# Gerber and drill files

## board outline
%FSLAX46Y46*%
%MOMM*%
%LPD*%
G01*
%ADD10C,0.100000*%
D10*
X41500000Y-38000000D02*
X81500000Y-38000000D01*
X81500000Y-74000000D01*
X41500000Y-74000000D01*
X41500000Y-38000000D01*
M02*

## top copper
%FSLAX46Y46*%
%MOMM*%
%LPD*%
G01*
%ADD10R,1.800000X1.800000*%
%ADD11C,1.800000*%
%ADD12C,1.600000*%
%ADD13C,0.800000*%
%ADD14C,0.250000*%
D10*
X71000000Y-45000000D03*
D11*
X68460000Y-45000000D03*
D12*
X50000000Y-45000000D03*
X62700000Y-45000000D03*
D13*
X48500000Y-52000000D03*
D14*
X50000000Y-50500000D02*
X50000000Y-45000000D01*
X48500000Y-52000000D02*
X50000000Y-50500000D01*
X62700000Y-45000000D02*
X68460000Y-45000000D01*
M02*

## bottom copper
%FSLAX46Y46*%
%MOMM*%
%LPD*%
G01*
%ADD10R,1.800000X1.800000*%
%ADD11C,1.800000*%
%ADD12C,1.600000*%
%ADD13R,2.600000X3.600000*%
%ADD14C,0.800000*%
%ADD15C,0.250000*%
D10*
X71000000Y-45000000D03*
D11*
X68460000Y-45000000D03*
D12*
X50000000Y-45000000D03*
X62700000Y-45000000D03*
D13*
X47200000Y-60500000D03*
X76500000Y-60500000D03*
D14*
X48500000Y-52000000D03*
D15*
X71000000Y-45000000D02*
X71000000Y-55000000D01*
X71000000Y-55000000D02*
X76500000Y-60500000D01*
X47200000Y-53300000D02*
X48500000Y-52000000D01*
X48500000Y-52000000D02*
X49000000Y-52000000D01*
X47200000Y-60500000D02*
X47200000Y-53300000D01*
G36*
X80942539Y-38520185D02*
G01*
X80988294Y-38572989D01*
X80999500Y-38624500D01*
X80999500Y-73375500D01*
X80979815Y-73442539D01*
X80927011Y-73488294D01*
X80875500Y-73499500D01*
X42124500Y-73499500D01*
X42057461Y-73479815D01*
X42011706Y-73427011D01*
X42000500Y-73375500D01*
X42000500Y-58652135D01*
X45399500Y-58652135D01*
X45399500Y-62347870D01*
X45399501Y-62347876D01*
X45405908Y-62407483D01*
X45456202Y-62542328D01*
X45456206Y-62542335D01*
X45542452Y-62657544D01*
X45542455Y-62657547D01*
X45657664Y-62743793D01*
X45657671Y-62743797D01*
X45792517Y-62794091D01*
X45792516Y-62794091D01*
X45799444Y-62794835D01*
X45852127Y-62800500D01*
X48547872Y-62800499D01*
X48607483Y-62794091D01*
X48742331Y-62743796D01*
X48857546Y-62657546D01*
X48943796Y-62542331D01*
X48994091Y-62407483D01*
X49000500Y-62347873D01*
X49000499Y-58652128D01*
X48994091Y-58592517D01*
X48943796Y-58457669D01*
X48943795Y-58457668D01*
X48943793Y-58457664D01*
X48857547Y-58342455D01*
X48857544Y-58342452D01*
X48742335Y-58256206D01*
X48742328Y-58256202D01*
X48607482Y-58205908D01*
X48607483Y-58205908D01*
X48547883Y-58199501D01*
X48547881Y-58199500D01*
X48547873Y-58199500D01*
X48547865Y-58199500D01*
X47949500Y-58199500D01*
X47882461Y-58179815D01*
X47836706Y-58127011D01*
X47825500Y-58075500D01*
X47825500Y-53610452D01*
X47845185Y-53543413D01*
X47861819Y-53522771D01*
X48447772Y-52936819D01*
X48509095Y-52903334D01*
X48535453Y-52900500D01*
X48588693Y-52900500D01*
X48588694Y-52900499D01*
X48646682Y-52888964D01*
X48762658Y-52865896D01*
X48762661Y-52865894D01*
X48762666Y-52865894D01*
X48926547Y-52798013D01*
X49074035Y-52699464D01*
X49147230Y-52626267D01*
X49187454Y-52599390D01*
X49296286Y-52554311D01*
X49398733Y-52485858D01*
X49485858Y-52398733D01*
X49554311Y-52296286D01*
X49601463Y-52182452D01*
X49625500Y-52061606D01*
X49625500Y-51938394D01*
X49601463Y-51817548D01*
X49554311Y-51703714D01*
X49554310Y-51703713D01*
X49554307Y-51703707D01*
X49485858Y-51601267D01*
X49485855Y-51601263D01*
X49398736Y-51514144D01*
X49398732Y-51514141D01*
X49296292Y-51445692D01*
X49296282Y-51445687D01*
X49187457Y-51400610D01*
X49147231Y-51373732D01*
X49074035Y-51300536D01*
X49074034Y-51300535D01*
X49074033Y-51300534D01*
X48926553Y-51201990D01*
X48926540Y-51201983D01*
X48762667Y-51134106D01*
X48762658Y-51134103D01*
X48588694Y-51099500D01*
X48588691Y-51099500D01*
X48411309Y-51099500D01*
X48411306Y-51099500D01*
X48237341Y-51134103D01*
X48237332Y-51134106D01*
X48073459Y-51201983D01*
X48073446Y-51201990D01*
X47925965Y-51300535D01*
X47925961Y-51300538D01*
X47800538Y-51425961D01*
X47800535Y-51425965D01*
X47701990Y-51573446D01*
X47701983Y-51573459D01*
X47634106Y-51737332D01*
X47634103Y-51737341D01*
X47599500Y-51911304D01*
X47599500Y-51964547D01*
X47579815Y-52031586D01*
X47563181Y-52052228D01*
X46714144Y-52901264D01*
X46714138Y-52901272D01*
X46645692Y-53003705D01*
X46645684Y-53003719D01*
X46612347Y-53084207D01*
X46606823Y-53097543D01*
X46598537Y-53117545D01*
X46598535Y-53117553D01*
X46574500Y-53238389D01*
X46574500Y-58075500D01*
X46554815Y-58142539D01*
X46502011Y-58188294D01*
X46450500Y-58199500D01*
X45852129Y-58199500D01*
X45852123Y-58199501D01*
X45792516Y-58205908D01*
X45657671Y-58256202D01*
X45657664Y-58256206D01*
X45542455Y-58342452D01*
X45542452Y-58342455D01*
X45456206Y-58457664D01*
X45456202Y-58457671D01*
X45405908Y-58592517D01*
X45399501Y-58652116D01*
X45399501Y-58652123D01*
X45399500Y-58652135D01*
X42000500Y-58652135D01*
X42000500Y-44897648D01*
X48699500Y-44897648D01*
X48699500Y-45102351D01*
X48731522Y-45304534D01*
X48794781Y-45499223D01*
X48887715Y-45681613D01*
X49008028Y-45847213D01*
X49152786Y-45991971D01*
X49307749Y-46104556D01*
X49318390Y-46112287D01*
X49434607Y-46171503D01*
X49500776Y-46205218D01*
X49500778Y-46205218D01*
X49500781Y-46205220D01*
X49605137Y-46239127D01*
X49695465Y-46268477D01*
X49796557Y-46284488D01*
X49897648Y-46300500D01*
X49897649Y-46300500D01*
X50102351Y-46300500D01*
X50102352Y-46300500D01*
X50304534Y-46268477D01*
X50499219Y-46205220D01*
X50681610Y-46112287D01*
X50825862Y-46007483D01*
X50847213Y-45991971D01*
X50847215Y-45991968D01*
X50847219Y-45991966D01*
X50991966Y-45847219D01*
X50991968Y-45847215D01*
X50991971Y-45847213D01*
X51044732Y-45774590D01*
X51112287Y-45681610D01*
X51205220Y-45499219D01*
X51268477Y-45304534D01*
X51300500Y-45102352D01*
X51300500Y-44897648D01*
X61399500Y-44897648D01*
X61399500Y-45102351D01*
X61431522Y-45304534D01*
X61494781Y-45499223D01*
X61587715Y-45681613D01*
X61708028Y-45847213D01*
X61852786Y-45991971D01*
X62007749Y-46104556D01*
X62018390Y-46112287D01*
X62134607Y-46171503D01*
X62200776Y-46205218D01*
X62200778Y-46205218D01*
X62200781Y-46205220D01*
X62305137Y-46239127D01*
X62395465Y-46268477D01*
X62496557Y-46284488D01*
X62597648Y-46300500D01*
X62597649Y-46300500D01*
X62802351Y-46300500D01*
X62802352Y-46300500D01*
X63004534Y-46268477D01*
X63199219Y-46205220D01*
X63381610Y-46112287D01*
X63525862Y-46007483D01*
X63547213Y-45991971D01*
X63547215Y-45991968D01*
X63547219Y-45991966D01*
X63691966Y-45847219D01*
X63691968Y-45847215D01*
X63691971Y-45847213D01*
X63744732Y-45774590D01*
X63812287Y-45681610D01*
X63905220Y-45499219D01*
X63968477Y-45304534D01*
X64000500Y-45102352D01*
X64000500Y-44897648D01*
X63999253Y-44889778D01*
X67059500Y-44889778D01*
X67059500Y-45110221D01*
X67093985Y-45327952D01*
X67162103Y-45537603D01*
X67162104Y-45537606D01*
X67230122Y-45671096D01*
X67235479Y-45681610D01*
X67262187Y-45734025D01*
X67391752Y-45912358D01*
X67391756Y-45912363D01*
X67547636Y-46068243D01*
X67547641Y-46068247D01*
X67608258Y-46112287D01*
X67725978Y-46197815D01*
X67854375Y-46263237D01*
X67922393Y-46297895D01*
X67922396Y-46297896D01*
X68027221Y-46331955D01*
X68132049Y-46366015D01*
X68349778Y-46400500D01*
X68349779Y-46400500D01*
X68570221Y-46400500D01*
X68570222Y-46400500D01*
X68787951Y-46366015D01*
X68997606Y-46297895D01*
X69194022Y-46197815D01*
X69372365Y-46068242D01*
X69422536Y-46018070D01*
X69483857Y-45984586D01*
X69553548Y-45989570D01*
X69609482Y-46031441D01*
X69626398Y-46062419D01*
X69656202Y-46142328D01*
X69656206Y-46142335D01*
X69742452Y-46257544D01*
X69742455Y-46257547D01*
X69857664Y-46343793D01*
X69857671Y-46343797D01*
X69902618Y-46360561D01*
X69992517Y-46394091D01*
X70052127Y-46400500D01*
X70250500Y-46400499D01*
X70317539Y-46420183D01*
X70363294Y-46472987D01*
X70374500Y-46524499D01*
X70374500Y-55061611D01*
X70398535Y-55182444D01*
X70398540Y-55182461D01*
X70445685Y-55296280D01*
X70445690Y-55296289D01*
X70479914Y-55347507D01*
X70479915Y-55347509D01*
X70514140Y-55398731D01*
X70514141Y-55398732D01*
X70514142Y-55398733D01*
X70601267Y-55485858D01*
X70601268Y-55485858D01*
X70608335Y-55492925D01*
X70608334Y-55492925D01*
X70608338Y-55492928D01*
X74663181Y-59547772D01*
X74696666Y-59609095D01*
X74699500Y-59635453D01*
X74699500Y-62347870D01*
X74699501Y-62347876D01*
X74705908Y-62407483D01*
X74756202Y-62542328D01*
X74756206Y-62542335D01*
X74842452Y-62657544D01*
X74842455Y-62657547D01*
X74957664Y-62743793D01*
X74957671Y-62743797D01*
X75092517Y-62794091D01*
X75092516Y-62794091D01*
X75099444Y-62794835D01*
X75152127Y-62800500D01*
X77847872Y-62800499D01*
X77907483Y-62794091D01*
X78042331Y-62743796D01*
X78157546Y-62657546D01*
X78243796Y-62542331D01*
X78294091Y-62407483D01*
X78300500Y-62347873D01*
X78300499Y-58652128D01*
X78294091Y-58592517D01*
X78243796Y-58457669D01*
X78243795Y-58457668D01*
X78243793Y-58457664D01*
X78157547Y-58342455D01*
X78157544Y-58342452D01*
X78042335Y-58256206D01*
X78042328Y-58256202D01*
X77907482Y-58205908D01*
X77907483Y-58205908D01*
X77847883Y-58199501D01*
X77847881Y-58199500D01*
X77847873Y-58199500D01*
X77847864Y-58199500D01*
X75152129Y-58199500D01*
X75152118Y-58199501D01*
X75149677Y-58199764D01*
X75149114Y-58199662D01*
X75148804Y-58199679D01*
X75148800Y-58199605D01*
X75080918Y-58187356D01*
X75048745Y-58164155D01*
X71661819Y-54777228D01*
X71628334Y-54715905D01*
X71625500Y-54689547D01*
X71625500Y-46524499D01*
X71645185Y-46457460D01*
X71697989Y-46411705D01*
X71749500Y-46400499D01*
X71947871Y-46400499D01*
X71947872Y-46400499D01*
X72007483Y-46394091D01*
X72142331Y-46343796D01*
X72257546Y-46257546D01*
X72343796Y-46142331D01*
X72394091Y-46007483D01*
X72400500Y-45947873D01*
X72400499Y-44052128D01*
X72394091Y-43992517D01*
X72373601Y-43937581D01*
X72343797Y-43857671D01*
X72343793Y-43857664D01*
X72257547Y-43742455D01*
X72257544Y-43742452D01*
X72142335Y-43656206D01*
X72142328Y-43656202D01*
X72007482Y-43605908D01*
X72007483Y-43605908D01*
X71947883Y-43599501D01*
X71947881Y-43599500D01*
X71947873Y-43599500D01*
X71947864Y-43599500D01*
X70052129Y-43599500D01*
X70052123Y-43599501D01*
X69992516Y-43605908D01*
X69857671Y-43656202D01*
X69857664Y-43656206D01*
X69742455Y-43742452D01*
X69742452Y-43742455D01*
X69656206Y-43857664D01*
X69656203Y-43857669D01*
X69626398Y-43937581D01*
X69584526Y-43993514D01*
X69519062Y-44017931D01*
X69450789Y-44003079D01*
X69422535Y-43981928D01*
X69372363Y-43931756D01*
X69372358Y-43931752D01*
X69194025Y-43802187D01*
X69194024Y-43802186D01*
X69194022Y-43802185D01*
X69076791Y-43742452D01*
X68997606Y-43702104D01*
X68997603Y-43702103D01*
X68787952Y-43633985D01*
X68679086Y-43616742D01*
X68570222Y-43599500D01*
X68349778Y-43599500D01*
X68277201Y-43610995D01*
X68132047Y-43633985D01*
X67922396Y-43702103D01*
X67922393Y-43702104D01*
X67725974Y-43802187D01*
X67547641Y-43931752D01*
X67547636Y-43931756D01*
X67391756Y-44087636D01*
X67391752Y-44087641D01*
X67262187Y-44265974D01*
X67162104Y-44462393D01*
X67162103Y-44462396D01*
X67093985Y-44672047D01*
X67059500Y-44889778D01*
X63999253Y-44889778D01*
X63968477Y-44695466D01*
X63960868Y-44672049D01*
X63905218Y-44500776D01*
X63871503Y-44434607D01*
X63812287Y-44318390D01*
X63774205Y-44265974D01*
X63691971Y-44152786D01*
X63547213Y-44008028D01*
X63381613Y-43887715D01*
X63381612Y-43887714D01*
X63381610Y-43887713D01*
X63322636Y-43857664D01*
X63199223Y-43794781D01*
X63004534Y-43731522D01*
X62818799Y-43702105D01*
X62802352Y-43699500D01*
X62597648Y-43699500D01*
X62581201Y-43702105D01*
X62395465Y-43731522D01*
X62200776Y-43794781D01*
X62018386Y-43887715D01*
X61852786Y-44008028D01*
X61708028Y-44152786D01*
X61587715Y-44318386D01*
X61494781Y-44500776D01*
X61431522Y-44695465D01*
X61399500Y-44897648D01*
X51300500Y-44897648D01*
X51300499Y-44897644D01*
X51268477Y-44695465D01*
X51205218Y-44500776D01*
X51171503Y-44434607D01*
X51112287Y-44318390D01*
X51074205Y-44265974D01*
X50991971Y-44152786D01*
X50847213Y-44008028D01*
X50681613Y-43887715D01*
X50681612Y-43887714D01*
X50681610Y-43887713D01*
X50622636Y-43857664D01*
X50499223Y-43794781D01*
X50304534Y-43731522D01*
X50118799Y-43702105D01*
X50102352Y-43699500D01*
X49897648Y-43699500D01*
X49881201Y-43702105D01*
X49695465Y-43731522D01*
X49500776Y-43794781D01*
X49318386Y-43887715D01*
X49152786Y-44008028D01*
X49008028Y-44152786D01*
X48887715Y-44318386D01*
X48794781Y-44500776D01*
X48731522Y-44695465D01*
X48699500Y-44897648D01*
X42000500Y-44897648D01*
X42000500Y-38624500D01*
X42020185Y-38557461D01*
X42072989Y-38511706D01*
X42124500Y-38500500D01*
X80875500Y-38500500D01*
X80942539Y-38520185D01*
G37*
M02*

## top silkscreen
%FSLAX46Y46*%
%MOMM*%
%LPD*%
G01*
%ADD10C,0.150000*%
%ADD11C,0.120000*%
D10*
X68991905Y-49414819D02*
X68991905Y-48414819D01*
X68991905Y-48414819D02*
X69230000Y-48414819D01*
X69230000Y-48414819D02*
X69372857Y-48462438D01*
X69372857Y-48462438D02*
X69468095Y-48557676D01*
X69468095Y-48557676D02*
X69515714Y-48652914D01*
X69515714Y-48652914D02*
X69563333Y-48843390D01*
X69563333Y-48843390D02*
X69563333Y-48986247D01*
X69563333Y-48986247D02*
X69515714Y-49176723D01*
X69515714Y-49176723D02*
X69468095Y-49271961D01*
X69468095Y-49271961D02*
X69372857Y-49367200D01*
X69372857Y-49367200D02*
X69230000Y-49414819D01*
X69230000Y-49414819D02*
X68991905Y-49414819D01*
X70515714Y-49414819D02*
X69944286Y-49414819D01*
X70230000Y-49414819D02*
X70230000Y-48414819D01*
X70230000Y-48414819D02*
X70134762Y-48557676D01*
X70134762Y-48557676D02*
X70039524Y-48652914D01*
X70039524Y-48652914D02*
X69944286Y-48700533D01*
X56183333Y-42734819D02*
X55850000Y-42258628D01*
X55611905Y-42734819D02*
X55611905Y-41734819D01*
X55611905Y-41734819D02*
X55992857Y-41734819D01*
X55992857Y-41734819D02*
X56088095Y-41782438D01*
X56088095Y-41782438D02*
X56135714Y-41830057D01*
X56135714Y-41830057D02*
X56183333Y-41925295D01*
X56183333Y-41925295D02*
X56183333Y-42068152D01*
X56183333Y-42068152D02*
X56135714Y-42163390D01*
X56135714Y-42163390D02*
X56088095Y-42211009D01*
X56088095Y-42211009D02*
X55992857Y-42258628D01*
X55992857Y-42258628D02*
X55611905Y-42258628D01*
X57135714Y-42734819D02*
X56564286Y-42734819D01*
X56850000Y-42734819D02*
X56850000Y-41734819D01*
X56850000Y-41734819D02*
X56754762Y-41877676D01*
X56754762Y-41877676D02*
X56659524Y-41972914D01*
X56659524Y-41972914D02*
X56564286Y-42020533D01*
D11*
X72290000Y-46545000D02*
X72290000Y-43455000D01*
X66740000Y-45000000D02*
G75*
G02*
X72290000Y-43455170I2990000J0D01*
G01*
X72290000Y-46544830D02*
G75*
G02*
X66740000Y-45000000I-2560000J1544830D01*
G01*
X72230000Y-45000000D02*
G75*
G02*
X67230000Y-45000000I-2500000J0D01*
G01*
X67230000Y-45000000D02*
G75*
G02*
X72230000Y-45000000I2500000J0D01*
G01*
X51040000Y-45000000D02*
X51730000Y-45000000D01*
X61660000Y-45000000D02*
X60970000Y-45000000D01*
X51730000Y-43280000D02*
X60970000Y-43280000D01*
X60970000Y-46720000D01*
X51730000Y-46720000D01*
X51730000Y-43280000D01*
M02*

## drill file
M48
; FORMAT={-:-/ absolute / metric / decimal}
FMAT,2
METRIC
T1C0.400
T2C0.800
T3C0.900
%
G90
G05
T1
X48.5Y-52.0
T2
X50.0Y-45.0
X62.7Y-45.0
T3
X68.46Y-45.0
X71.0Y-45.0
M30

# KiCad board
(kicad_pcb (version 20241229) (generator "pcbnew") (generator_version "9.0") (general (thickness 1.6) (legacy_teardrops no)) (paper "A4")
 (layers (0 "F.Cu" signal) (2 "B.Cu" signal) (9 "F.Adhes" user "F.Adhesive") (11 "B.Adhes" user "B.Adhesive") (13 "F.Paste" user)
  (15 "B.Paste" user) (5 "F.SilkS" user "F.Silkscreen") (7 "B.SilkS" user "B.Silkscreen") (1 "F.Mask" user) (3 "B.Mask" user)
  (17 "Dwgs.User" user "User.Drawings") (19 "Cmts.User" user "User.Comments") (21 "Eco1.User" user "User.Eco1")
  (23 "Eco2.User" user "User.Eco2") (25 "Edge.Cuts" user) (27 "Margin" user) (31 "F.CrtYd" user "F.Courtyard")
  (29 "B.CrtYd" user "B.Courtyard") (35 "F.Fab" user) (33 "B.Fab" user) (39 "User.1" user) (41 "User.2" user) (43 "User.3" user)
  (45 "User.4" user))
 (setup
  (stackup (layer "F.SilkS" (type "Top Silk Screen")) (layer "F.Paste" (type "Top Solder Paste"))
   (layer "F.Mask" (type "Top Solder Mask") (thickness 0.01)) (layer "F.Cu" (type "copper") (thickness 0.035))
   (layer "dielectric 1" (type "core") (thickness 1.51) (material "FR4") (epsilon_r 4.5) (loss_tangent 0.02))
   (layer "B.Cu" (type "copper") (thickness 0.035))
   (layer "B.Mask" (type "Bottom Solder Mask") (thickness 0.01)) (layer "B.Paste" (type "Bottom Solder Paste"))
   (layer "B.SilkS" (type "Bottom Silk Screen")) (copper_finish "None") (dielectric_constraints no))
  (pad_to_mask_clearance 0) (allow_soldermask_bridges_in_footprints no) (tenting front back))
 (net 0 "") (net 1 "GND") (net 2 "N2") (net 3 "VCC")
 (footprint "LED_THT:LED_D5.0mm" (layer "F.Cu") (at 71 45 180)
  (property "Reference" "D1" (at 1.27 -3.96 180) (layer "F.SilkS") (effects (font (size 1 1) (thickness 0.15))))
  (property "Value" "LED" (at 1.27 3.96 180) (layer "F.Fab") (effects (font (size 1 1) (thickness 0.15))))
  (fp_line (start -1.29 -1.545) (end -1.29 1.545) (stroke (width 0.12) (type solid)) (layer "F.SilkS"))
  (fp_arc (start 4.26 0) (mid 2.071779 2.880495) (end -1.29 1.54483) (stroke (width 0.12) (type solid)) (layer "F.SilkS"))
  (fp_arc (start -1.29 -1.54483) (mid 2.071779 -2.880495) (end 4.26 0) (stroke (width 0.12) (type solid)) (layer "F.SilkS"))
  (fp_circle (center 1.27 0) (end 3.77 0) (stroke (width 0.12) (type solid)) (fill no) (layer "F.SilkS"))
  (pad "1" thru_hole rect (at 0 0 180) (size 1.8 1.8) (drill 0.9) (layers "*.Cu" "*.Mask") (remove_unused_layers no) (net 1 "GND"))
  (pad "2" thru_hole circle (at 2.54 0 180) (size 1.8 1.8) (drill 0.9) (layers "*.Cu" "*.Mask") (remove_unused_layers no) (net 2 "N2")))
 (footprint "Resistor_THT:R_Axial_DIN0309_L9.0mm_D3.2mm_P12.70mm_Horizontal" (layer "F.Cu") (at 50 45)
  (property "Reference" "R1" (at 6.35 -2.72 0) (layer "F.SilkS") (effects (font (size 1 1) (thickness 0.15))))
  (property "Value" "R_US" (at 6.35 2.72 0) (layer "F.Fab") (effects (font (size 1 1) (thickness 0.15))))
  (fp_line (start 1.04 0) (end 1.73 0) (stroke (width 0.12) (type solid)) (layer "F.SilkS"))
  (fp_line (start 11.66 0) (end 10.97 0) (stroke (width 0.12) (type solid)) (layer "F.SilkS"))
  (fp_rect (start 1.73 -1.72) (end 10.97 1.72) (stroke (width 0.12) (type solid)) (fill no) (layer "F.SilkS"))
  (pad "1" thru_hole circle (at 0 0) (size 1.6 1.6) (drill 0.8) (layers "*.Cu" "*.Mask") (remove_unused_layers no) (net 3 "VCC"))
  (pad "2" thru_hole circle (at 12.7 0) (size 1.6 1.6) (drill 0.8) (layers "*.Cu" "*.Mask") (remove_unused_layers no) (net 2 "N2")))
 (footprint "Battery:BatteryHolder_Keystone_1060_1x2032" (layer "B.Cu") (at 61.85 60.5)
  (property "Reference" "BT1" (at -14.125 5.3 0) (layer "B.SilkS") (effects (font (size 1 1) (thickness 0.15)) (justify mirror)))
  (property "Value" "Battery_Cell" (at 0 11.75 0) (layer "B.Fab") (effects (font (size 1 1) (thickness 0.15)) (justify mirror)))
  (pad "1" smd rect (at -14.65 0 180) (size 2.6 3.6) (layers "B.Cu" "B.Mask" "B.Paste") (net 3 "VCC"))
  (pad "2" smd rect (at 14.65 0 180) (size 2.6 3.6) (layers "B.Cu" "B.Mask" "B.Paste") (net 1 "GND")))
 (gr_rect (start 41.5 38) (end 81.5 74) (stroke (width 0.1) (type default)) (fill no) (layer "Edge.Cuts"))
 (segment (start 71 45) (end 71 55) (width 0.25) (layer "B.Cu") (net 1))
 (segment (start 71 55) (end 76.5 60.5) (width 0.25) (layer "B.Cu") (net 1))
 (segment (start 50 50.5) (end 50 45) (width 0.25) (layer "F.Cu") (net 3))
 (segment (start 48.5 52) (end 50 50.5) (width 0.25) (layer "F.Cu") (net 3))
 (via (at 48.5 52) (size 0.8) (drill 0.4) (layers "F.Cu" "B.Cu") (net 3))
 (segment (start 47.2 53.3) (end 48.5 52) (width 0.25) (layer "B.Cu") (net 3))
 (segment (start 48.5 52) (end 49 52) (width 0.25) (layer "B.Cu") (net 3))
 (segment (start 47.2 60.5) (end 47.2 53.3) (width 0.25) (layer "B.Cu") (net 3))
 (segment (start 62.7 45) (end 68.46 45) (width 0.25) (layer "F.Cu") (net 2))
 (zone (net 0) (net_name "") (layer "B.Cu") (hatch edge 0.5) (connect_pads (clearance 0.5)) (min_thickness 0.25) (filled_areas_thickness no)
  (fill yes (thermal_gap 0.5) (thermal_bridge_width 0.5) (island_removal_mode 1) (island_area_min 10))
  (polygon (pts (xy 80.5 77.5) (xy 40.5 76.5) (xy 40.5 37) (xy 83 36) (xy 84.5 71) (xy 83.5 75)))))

